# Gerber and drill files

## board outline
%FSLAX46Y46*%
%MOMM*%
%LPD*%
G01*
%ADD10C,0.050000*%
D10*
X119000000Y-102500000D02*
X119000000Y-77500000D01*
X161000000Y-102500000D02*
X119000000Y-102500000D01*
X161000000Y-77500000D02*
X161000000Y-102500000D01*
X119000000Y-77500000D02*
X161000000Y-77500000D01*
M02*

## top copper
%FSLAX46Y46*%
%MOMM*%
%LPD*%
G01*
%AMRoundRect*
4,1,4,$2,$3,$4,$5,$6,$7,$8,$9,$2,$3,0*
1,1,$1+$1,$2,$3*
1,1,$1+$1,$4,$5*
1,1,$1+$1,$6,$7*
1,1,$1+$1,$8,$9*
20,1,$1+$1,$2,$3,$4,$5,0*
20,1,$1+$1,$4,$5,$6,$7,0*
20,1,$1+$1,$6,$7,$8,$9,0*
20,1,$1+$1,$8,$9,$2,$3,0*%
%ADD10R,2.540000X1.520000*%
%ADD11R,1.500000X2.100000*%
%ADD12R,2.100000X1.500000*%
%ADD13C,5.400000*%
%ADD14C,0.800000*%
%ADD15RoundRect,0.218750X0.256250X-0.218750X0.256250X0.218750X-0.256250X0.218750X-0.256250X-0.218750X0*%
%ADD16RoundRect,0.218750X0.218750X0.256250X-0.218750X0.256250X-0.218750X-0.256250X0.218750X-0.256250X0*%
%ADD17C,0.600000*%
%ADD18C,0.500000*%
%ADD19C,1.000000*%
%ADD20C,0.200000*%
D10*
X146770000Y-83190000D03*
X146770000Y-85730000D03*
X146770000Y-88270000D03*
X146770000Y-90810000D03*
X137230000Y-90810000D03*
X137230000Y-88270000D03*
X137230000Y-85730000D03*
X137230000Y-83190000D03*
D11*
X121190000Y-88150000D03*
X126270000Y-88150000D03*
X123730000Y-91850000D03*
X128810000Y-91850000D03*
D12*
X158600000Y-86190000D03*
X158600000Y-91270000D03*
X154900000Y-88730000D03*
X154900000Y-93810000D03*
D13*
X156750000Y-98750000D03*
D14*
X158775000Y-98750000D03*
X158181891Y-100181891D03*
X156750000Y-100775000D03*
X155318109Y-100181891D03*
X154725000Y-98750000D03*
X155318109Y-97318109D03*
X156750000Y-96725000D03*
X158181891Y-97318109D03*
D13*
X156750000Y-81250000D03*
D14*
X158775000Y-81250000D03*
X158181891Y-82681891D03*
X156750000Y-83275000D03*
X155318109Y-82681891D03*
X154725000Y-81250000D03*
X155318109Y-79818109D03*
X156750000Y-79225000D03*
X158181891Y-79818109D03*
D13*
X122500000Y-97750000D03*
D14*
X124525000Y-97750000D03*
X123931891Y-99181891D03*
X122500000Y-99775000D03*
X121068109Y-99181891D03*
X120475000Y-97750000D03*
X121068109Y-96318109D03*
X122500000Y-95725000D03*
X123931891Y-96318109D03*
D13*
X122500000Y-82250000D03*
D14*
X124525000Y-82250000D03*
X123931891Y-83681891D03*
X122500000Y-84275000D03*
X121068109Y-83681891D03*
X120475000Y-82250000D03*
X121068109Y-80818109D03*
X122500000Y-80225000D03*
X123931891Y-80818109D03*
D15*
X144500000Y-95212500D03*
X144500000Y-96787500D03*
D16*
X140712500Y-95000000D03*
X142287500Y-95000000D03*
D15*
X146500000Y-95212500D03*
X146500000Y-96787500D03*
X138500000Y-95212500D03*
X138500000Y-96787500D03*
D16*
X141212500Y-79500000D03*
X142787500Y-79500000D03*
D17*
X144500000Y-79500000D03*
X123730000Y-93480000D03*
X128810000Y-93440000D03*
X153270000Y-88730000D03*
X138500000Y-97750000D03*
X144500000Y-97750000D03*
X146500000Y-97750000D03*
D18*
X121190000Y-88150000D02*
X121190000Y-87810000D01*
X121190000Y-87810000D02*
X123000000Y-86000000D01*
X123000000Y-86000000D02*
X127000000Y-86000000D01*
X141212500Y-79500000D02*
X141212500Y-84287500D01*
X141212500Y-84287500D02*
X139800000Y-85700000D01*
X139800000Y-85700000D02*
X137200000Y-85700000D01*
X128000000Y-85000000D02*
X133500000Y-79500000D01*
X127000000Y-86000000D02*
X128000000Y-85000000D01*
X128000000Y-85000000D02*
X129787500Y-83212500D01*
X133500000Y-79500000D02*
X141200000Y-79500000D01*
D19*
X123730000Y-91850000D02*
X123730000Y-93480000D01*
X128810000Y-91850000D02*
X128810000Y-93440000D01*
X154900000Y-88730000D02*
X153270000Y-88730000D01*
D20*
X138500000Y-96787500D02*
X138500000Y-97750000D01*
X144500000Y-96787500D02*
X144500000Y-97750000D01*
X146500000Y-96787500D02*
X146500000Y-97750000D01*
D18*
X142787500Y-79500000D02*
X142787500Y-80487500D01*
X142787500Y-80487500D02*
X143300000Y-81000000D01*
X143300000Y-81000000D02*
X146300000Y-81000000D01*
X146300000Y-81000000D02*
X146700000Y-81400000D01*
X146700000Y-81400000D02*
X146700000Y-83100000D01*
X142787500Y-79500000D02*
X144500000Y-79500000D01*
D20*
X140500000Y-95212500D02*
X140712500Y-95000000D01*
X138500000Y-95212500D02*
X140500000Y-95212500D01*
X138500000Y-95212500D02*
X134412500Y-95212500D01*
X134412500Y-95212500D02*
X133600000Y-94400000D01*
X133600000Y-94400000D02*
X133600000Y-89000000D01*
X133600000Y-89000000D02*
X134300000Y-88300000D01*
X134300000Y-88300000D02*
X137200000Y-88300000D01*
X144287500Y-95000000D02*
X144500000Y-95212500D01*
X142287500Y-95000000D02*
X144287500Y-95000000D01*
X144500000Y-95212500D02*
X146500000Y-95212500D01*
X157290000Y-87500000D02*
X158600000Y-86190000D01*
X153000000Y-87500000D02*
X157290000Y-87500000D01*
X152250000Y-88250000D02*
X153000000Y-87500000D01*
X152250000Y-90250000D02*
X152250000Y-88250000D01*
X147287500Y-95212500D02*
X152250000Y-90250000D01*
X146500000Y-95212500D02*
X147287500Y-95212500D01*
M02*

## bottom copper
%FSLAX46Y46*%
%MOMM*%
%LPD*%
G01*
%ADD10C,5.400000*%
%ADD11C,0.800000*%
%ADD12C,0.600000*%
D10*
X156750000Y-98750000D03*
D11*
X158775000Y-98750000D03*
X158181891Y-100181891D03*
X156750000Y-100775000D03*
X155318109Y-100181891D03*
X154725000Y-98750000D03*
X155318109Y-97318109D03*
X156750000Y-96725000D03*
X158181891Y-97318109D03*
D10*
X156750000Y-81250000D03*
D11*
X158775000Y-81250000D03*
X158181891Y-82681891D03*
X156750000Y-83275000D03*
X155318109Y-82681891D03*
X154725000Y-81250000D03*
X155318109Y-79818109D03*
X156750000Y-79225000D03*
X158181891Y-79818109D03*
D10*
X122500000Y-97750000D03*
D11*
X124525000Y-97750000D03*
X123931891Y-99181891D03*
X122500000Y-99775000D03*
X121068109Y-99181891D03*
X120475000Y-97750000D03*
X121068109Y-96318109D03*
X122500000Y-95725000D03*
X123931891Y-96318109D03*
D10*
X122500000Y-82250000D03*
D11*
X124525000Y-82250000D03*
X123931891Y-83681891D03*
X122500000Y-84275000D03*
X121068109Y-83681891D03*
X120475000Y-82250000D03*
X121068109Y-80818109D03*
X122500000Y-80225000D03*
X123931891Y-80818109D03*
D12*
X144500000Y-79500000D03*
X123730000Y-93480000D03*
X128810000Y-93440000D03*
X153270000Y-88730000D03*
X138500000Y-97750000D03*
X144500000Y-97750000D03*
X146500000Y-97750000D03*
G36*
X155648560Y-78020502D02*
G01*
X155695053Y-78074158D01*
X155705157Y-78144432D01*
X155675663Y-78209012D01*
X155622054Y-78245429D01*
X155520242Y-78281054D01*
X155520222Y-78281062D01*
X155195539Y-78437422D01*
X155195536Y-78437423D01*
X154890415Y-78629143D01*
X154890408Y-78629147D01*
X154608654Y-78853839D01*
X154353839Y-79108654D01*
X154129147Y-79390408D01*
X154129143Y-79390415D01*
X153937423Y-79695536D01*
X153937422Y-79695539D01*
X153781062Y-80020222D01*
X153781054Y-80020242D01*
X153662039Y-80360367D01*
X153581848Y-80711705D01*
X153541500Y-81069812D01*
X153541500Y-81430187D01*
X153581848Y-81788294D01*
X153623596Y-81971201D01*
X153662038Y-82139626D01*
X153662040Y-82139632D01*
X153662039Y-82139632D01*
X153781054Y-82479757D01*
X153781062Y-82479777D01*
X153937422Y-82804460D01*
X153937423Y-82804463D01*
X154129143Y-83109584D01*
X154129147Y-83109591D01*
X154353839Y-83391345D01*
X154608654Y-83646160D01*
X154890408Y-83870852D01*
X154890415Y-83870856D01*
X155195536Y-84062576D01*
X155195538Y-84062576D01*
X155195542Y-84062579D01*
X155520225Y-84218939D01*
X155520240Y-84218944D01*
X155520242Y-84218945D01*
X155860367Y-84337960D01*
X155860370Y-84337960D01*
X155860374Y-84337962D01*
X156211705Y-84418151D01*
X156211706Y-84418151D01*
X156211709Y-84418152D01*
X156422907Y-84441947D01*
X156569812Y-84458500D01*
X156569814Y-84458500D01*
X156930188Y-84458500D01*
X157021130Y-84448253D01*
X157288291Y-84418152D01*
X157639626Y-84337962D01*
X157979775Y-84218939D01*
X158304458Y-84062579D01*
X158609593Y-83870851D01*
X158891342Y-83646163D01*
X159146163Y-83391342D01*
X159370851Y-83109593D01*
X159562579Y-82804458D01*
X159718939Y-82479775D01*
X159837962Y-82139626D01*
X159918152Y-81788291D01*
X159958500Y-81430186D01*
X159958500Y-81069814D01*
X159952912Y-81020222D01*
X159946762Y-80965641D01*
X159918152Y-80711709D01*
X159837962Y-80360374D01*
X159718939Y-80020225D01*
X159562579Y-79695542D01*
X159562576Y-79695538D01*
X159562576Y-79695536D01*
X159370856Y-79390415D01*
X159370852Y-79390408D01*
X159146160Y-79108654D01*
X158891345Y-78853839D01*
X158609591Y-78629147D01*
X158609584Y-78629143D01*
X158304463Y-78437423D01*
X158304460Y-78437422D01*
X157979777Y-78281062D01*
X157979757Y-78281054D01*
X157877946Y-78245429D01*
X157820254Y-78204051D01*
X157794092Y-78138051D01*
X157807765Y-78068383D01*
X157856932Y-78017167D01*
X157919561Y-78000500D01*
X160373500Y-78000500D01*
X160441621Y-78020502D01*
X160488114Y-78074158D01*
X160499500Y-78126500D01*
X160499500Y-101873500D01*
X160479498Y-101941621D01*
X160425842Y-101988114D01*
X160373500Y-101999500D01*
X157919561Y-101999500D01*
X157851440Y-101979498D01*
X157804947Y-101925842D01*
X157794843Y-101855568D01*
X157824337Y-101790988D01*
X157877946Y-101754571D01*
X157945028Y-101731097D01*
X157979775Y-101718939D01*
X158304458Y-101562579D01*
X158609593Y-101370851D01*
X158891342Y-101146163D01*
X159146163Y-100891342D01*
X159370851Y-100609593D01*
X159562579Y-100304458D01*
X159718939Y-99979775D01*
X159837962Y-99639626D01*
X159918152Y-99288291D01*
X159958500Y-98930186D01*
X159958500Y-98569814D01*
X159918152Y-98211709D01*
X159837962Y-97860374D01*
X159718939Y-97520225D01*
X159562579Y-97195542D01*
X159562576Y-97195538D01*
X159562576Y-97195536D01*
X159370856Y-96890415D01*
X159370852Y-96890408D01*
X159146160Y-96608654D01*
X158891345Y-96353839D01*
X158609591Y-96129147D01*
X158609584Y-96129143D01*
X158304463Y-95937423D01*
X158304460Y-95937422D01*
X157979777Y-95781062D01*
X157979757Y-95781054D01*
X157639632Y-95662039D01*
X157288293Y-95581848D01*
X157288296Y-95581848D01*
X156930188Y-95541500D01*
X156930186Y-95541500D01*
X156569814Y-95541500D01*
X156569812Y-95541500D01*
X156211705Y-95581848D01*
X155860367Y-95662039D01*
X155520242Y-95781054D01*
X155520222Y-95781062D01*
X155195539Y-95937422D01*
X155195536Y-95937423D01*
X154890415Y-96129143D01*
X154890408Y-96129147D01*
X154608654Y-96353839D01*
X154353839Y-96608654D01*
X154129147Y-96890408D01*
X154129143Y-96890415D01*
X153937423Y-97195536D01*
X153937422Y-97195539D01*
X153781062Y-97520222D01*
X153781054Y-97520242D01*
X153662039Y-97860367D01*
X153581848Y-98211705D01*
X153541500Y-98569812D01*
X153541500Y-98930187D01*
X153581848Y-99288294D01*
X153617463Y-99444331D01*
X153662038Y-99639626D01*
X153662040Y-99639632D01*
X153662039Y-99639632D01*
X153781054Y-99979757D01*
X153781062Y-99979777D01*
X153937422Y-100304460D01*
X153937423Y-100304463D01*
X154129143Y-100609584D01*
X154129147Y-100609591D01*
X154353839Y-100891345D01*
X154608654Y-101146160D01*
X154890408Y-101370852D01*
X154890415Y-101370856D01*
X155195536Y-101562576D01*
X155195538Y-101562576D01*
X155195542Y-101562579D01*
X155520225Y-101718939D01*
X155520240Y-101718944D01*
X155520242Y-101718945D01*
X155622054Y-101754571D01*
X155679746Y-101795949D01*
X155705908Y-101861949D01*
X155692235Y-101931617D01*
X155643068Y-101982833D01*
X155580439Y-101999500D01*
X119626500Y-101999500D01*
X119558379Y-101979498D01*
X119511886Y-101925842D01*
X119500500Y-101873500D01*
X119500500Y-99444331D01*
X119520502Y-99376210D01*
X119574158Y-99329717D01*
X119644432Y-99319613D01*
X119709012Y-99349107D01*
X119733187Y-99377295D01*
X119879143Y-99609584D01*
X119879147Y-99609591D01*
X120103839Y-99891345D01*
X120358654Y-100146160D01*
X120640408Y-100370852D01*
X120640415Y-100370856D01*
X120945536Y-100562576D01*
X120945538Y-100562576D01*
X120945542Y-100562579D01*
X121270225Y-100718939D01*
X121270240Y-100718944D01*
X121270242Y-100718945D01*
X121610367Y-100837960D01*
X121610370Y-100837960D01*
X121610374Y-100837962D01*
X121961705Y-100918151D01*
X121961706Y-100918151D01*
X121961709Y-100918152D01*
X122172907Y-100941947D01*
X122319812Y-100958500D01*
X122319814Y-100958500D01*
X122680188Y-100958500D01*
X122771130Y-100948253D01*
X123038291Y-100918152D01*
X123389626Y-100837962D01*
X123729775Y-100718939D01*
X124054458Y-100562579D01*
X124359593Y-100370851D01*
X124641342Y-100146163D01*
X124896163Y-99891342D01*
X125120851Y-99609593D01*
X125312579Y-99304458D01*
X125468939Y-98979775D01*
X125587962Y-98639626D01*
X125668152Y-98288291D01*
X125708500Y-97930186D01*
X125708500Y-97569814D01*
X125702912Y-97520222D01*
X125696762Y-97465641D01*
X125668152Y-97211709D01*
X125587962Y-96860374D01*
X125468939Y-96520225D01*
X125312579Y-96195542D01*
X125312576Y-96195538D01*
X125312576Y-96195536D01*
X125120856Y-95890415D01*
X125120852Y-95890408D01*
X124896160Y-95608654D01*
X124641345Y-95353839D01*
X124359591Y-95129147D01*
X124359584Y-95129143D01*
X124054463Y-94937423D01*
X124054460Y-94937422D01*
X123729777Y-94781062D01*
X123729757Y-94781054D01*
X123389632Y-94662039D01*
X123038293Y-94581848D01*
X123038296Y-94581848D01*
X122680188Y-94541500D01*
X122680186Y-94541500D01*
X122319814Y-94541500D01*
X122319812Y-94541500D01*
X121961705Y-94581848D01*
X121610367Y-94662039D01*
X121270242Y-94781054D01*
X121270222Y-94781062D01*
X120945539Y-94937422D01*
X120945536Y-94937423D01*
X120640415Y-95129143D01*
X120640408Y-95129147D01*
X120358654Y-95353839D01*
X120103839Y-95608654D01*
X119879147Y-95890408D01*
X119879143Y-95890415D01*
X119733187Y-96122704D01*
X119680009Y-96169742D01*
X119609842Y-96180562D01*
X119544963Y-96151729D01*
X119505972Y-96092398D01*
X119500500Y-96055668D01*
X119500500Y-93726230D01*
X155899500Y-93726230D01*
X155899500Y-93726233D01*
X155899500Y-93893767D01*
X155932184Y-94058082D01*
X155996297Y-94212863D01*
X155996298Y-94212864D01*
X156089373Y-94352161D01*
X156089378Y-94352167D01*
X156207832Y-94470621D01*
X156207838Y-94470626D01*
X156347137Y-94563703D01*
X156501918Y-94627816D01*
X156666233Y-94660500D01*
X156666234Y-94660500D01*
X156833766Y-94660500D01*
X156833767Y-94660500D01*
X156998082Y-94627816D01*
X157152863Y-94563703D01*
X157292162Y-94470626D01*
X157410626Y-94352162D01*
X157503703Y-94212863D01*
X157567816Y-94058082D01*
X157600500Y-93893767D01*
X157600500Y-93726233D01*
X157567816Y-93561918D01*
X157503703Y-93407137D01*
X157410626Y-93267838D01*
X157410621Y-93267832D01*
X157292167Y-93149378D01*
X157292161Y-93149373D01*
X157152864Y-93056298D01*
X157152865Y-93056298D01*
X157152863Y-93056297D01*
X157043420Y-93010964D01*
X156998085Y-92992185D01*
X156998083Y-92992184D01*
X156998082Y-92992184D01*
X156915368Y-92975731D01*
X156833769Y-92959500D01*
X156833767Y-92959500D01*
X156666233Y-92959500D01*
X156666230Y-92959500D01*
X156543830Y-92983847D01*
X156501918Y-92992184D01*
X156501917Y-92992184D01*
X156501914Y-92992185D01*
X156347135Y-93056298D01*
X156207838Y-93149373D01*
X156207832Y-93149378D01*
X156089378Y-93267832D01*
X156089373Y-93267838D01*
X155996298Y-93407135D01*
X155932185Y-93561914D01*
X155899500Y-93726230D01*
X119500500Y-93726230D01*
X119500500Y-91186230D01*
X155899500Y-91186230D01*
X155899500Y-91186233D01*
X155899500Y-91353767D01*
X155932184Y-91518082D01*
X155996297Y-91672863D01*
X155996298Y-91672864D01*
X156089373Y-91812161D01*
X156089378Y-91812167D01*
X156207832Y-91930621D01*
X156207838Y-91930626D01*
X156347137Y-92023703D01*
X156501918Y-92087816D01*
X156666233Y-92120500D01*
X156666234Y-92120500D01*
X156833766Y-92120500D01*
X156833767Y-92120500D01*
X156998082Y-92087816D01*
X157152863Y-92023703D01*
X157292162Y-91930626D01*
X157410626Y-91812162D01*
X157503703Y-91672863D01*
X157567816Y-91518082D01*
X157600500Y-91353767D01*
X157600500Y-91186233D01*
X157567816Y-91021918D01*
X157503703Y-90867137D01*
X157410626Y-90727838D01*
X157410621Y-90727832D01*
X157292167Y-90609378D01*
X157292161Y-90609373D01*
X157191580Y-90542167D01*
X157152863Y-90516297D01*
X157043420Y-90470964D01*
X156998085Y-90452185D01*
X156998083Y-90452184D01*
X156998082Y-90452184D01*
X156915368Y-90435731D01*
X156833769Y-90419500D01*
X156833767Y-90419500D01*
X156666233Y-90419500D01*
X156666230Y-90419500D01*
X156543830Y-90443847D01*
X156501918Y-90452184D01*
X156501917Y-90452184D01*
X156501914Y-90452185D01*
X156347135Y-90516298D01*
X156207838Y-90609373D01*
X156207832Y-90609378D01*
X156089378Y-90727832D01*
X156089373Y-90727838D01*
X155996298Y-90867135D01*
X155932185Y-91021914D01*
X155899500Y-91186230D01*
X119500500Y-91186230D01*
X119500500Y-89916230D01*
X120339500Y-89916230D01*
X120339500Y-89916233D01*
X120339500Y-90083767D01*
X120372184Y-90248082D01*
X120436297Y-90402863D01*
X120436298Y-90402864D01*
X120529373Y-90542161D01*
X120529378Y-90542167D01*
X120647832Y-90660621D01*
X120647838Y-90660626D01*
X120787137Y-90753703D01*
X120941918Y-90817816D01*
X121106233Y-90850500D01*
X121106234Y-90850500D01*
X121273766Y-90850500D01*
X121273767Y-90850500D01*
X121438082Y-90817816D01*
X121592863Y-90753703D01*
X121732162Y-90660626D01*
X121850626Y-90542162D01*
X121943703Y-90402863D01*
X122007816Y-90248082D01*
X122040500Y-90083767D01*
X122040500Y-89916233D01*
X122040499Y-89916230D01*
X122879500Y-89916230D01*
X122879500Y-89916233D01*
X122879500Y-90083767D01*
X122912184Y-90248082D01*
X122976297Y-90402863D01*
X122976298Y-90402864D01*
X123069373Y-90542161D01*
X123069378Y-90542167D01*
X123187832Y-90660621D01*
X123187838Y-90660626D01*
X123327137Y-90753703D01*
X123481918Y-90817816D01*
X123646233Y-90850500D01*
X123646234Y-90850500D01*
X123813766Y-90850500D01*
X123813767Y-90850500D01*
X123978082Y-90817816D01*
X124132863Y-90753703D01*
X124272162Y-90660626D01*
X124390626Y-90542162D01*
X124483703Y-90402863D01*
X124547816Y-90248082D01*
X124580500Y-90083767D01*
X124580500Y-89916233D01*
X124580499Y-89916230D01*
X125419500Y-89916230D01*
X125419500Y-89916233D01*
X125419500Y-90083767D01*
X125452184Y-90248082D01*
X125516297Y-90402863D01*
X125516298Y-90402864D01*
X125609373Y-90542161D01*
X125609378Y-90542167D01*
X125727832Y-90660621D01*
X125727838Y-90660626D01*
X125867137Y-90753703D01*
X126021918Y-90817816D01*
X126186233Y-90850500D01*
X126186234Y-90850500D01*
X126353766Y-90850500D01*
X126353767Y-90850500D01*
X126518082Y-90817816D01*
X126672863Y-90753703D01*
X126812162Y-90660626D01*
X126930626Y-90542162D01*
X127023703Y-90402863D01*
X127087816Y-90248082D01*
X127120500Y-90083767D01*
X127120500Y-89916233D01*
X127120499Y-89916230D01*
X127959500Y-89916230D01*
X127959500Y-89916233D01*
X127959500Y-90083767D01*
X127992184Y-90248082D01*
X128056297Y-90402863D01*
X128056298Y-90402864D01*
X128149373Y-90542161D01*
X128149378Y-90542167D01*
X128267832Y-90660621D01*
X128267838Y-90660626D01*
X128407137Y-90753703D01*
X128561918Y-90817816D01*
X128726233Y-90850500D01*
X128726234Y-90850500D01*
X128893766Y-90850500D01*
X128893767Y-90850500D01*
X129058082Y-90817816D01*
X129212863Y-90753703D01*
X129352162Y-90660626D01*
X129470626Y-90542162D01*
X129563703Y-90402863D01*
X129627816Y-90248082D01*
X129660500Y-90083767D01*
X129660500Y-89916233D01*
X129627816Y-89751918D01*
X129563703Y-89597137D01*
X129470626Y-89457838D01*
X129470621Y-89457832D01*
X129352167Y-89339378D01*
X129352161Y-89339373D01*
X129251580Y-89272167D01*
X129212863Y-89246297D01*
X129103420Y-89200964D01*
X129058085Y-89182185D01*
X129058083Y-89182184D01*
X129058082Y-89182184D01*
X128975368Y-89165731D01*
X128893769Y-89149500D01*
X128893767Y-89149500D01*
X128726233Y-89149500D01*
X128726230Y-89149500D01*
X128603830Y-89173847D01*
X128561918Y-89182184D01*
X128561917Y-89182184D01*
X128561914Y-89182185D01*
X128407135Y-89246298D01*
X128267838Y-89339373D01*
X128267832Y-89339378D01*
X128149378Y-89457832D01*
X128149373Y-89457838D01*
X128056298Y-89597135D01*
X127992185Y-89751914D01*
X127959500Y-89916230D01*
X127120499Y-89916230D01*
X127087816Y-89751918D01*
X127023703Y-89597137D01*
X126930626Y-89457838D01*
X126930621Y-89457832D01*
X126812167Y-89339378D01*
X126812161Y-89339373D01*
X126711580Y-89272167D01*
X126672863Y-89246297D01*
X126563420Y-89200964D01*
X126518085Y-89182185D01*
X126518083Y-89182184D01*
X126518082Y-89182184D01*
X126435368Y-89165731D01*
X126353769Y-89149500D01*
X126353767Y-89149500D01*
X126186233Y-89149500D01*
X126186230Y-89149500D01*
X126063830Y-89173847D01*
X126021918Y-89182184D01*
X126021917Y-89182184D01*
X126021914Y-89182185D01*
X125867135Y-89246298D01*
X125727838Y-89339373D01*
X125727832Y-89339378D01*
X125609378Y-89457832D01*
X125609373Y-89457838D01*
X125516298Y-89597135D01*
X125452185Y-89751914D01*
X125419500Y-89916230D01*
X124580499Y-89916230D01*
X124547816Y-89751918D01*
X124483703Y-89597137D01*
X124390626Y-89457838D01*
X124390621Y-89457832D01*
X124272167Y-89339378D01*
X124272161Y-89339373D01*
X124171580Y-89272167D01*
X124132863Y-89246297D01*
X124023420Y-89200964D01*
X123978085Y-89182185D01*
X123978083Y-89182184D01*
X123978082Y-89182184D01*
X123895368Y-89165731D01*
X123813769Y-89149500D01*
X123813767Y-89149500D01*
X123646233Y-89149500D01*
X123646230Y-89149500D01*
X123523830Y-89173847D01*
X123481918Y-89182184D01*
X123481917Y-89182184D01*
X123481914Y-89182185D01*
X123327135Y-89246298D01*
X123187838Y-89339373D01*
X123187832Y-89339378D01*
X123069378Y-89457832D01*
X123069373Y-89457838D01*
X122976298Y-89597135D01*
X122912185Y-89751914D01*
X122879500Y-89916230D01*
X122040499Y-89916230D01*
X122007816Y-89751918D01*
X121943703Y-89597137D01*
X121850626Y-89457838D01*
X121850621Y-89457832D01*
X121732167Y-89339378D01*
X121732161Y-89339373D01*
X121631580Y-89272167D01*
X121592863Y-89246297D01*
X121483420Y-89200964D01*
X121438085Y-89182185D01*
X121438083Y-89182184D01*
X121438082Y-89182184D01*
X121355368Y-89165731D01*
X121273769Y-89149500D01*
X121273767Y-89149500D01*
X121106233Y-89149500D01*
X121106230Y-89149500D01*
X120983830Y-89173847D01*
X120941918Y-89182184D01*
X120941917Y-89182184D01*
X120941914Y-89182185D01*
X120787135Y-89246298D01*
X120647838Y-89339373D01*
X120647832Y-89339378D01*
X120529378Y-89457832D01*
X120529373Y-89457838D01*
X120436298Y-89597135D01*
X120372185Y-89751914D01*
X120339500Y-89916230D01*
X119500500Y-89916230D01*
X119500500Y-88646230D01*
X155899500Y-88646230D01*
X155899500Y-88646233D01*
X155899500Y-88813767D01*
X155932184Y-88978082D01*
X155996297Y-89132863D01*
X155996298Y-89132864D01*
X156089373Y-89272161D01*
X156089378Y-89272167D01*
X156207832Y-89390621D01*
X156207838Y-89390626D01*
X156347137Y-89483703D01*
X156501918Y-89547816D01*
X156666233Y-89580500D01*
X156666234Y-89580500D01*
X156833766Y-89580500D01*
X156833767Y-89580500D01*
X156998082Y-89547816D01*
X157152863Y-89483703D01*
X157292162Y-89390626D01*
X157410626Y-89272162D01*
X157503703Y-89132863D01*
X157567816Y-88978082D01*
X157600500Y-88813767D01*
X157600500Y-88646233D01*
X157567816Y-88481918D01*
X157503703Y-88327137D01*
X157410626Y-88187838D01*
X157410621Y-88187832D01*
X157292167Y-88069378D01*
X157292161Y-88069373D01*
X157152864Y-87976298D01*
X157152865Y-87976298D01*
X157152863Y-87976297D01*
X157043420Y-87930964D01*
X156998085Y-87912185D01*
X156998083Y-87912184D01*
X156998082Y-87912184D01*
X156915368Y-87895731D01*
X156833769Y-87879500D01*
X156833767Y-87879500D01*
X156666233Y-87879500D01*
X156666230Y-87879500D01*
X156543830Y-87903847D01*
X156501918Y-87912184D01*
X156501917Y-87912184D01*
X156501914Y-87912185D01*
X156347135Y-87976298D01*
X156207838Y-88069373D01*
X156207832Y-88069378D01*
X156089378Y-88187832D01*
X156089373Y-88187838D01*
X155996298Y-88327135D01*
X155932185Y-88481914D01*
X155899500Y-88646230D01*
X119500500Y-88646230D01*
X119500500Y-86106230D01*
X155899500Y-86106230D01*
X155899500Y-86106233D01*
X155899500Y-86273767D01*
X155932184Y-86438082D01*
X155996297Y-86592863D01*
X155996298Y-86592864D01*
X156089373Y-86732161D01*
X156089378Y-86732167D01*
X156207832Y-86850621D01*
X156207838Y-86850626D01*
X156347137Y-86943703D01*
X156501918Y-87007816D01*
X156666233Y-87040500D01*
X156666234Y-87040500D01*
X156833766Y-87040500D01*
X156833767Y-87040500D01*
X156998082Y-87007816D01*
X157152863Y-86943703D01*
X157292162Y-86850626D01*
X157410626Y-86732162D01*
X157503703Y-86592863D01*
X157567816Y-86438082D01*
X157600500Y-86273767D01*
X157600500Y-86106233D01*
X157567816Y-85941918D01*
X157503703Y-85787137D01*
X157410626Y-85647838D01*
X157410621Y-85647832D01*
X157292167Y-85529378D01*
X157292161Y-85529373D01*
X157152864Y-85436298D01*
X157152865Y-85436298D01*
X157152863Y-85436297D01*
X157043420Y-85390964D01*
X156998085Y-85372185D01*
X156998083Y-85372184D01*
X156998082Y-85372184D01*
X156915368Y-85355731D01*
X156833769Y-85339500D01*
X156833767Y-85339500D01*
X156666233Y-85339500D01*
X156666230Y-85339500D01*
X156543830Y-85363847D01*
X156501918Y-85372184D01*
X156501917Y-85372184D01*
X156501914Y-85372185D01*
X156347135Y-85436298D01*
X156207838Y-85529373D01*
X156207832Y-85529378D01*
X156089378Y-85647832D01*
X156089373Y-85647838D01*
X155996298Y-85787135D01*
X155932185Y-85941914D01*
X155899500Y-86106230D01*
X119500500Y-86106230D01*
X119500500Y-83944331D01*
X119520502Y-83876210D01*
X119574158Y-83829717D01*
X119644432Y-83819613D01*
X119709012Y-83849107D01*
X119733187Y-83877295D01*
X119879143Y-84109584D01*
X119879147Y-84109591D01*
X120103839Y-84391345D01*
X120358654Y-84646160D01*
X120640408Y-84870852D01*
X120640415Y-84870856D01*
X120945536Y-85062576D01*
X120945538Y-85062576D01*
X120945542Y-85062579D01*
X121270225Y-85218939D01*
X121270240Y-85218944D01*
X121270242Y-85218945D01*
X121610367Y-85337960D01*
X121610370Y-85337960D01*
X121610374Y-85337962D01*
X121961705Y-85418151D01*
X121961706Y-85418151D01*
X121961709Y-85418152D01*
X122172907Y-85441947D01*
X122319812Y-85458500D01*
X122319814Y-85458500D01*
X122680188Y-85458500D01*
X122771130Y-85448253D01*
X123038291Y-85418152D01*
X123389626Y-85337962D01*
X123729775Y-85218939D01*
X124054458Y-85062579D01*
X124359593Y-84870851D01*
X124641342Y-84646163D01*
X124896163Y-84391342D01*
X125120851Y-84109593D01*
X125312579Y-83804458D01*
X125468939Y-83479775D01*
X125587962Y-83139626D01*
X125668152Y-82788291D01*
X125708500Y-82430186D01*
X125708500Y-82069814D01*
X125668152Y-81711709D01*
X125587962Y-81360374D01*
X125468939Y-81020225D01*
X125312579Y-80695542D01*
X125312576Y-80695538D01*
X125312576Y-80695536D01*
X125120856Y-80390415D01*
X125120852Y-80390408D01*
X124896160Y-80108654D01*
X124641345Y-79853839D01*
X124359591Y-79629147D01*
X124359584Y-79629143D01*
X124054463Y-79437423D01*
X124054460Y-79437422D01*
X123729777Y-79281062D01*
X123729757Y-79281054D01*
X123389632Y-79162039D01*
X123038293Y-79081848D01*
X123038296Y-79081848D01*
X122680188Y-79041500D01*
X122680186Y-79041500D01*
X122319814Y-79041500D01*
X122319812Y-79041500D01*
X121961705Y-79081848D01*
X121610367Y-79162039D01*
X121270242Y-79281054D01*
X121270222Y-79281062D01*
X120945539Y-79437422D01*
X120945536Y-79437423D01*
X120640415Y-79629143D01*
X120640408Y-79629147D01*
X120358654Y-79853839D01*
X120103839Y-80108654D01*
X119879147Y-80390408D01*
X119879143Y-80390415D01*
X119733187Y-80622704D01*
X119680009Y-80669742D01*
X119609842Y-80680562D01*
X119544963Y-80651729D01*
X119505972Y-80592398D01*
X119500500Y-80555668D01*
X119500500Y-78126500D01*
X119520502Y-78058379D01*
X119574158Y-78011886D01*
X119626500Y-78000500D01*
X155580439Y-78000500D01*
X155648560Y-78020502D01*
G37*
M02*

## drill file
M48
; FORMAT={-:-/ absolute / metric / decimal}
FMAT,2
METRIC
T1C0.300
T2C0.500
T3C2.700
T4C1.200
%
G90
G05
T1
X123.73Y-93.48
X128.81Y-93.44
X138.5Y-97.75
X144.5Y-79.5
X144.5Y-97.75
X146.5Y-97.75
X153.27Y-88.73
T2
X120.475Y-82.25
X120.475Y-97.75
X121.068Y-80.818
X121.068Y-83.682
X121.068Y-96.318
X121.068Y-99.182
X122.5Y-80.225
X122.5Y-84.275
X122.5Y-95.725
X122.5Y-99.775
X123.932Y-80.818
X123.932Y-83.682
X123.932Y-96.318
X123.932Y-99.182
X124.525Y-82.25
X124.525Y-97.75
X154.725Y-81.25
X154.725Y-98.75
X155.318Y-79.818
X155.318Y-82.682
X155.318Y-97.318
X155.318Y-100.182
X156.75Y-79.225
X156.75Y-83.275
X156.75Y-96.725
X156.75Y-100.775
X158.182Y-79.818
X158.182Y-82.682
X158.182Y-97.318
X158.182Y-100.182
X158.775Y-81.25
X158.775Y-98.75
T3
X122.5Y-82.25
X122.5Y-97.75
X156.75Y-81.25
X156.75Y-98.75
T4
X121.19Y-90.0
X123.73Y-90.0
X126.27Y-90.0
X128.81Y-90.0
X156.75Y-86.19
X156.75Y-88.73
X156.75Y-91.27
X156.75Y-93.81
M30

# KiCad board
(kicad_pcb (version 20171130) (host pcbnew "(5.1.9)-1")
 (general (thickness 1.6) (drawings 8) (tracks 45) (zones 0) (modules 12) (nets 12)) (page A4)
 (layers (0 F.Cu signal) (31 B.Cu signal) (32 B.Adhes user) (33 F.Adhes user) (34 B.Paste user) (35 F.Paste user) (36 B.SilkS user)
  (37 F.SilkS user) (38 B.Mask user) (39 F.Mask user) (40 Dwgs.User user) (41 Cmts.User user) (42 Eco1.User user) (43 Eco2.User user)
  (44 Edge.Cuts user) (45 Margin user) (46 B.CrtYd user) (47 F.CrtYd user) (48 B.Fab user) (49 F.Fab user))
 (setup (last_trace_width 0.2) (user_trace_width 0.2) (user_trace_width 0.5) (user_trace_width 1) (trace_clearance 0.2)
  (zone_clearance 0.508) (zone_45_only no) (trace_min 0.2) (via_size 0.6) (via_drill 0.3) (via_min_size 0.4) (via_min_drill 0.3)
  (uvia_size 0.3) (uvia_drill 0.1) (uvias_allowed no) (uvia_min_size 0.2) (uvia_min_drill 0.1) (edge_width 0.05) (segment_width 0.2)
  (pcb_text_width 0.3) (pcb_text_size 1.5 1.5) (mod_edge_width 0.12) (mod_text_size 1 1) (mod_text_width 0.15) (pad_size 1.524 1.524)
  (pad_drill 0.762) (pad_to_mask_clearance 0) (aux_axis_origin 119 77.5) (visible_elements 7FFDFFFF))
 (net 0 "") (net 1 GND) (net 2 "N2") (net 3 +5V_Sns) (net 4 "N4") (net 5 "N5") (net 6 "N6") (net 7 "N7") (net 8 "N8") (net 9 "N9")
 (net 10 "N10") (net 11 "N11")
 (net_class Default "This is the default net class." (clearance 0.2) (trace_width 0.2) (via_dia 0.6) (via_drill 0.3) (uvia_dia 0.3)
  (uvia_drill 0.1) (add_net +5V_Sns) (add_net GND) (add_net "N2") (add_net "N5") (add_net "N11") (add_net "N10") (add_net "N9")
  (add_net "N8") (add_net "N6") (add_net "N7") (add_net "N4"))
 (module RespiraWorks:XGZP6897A (layer F.Cu) (at 142 87)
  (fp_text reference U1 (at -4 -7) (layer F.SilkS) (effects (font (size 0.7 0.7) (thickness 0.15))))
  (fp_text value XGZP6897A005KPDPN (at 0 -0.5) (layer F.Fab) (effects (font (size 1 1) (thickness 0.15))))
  (pad 8 smd rect (at 4.77 -3.81) (size 2.54 1.52) (layers F.Cu F.Paste F.Mask) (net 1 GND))
  (pad 7 smd rect (at 4.77 -1.27) (size 2.54 1.52) (layers F.Cu F.Paste F.Mask))
  (pad 6 smd rect (at 4.77 1.27) (size 2.54 1.52) (layers F.Cu F.Paste F.Mask))
  (pad 5 smd rect (at 4.77 3.81) (size 2.54 1.52) (layers F.Cu F.Paste F.Mask))
  (pad 4 smd rect (at -4.77 3.81) (size 2.54 1.52) (layers F.Cu F.Paste F.Mask))
  (pad 3 smd rect (at -4.77 1.27) (size 2.54 1.52) (layers F.Cu F.Paste F.Mask) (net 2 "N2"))
  (pad 2 smd rect (at -4.77 -1.27) (size 2.54 1.52) (layers F.Cu F.Paste F.Mask) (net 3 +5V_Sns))
  (pad 1 smd rect (at -4.77 -3.81) (size 2.54 1.52) (layers F.Cu F.Paste F.Mask)))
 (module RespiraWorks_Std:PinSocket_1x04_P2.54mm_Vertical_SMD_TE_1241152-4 (layer F.Cu) (at 125 90 90)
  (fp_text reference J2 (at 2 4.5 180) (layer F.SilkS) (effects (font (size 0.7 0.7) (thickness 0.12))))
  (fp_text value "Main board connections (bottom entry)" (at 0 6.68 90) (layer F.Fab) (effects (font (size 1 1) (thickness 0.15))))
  (pad "" np_thru_hole circle (at 0 1.27 90) (size 1.2 1.2) (drill 1.2) (layers *.Cu *.Mask))
  (pad "" np_thru_hole circle (at 0 -1.27 90) (size 1.2 1.2) (drill 1.2) (layers *.Cu *.Mask))
  (pad "" np_thru_hole circle (at 0 -3.81 90) (size 1.2 1.2) (drill 1.2) (layers *.Cu *.Mask))
  (pad 1 smd rect (at 1.85 -3.81 90) (size 2.1 1.5) (layers F.Cu F.Paste F.Mask) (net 3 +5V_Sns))
  (pad 3 smd rect (at 1.85 1.27 90) (size 2.1 1.5) (layers F.Cu F.Paste F.Mask) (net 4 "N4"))
  (pad 2 smd rect (at -1.85 -1.27 90) (size 2.1 1.5) (layers F.Cu F.Paste F.Mask) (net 1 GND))
  (pad 4 smd rect (at -1.85 3.81 90) (size 2.1 1.5) (layers F.Cu F.Paste F.Mask) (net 1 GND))
  (pad "" np_thru_hole circle (at 0 3.81 90) (size 1.2 1.2) (drill 1.2) (layers *.Cu *.Mask)))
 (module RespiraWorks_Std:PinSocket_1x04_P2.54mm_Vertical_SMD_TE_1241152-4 (layer F.Cu) (at 156.75 90)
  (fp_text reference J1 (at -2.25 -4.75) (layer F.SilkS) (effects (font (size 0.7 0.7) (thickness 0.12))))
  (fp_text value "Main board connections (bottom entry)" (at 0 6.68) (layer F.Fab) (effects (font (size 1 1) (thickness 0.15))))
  (pad "" np_thru_hole circle (at 0 1.27) (size 1.2 1.2) (drill 1.2) (layers *.Cu *.Mask))
  (pad "" np_thru_hole circle (at 0 -1.27) (size 1.2 1.2) (drill 1.2) (layers *.Cu *.Mask))
  (pad "" np_thru_hole circle (at 0 -3.81) (size 1.2 1.2) (drill 1.2) (layers *.Cu *.Mask))
  (pad 1 smd rect (at 1.85 -3.81) (size 2.1 1.5) (layers F.Cu F.Paste F.Mask) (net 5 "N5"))
  (pad 3 smd rect (at 1.85 1.27) (size 2.1 1.5) (layers F.Cu F.Paste F.Mask) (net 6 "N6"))
  (pad 2 smd rect (at -1.85 -1.27) (size 2.1 1.5) (layers F.Cu F.Paste F.Mask) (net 1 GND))
  (pad 4 smd rect (at -1.85 3.81) (size 2.1 1.5) (layers F.Cu F.Paste F.Mask) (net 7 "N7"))
  (pad "" np_thru_hole circle (at 0 3.81) (size 1.2 1.2) (drill 1.2) (layers *.Cu *.Mask)))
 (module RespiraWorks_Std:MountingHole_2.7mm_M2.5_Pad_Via (layer F.Cu) (at 156.75 98.75)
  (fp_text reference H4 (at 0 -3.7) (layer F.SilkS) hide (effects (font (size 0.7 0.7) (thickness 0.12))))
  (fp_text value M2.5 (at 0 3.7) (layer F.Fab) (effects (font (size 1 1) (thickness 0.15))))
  (pad 1 thru_hole circle (at 0 0) (size 5.4 5.4) (drill 2.7) (layers *.Cu *.Mask) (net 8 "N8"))
  (pad 1 thru_hole circle (at 2.025 0) (size 0.8 0.8) (drill 0.5) (layers *.Cu *.Mask) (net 8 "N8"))
  (pad 1 thru_hole circle (at 1.431891 1.431891) (size 0.8 0.8) (drill 0.5) (layers *.Cu *.Mask) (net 8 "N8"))
  (pad 1 thru_hole circle (at 0 2.025) (size 0.8 0.8) (drill 0.5) (layers *.Cu *.Mask) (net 8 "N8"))
  (pad 1 thru_hole circle (at -1.431891 1.431891) (size 0.8 0.8) (drill 0.5) (layers *.Cu *.Mask) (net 8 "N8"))
  (pad 1 thru_hole circle (at -2.025 0) (size 0.8 0.8) (drill 0.5) (layers *.Cu *.Mask) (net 8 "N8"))
  (pad 1 thru_hole circle (at -1.431891 -1.431891) (size 0.8 0.8) (drill 0.5) (layers *.Cu *.Mask) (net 8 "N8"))
  (pad 1 thru_hole circle (at 0 -2.025) (size 0.8 0.8) (drill 0.5) (layers *.Cu *.Mask) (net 8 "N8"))
  (pad 1 thru_hole circle (at 1.431891 -1.431891) (size 0.8 0.8) (drill 0.5) (layers *.Cu *.Mask) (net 8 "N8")))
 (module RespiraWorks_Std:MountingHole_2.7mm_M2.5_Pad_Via (layer F.Cu) (at 156.75 81.25)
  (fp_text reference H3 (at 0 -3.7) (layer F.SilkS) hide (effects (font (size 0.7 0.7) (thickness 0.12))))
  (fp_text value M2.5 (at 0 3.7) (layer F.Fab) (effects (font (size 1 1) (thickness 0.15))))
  (pad 1 thru_hole circle (at 0 0) (size 5.4 5.4) (drill 2.7) (layers *.Cu *.Mask) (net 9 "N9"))
  (pad 1 thru_hole circle (at 2.025 0) (size 0.8 0.8) (drill 0.5) (layers *.Cu *.Mask) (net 9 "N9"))
  (pad 1 thru_hole circle (at 1.431891 1.431891) (size 0.8 0.8) (drill 0.5) (layers *.Cu *.Mask) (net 9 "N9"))
  (pad 1 thru_hole circle (at 0 2.025) (size 0.8 0.8) (drill 0.5) (layers *.Cu *.Mask) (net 9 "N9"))
  (pad 1 thru_hole circle (at -1.431891 1.431891) (size 0.8 0.8) (drill 0.5) (layers *.Cu *.Mask) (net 9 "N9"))
  (pad 1 thru_hole circle (at -2.025 0) (size 0.8 0.8) (drill 0.5) (layers *.Cu *.Mask) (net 9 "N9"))
  (pad 1 thru_hole circle (at -1.431891 -1.431891) (size 0.8 0.8) (drill 0.5) (layers *.Cu *.Mask) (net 9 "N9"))
  (pad 1 thru_hole circle (at 0 -2.025) (size 0.8 0.8) (drill 0.5) (layers *.Cu *.Mask) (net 9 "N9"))
  (pad 1 thru_hole circle (at 1.431891 -1.431891) (size 0.8 0.8) (drill 0.5) (layers *.Cu *.Mask) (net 9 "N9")))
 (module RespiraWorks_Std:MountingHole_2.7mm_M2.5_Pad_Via (layer F.Cu) (at 122.5 97.75)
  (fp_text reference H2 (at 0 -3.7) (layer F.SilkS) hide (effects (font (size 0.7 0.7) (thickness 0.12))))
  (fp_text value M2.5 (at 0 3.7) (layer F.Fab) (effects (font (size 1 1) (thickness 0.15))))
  (pad 1 thru_hole circle (at 0 0) (size 5.4 5.4) (drill 2.7) (layers *.Cu *.Mask) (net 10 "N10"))
  (pad 1 thru_hole circle (at 2.025 0) (size 0.8 0.8) (drill 0.5) (layers *.Cu *.Mask) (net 10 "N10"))
  (pad 1 thru_hole circle (at 1.431891 1.431891) (size 0.8 0.8) (drill 0.5) (layers *.Cu *.Mask) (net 10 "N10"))
  (pad 1 thru_hole circle (at 0 2.025) (size 0.8 0.8) (drill 0.5) (layers *.Cu *.Mask) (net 10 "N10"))
  (pad 1 thru_hole circle (at -1.431891 1.431891) (size 0.8 0.8) (drill 0.5) (layers *.Cu *.Mask) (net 10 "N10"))
  (pad 1 thru_hole circle (at -2.025 0) (size 0.8 0.8) (drill 0.5) (layers *.Cu *.Mask) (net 10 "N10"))
  (pad 1 thru_hole circle (at -1.431891 -1.431891) (size 0.8 0.8) (drill 0.5) (layers *.Cu *.Mask) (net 10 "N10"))
  (pad 1 thru_hole circle (at 0 -2.025) (size 0.8 0.8) (drill 0.5) (layers *.Cu *.Mask) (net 10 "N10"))
  (pad 1 thru_hole circle (at 1.431891 -1.431891) (size 0.8 0.8) (drill 0.5) (layers *.Cu *.Mask) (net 10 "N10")))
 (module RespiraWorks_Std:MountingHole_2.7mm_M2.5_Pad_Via (layer F.Cu) (at 122.5 82.25)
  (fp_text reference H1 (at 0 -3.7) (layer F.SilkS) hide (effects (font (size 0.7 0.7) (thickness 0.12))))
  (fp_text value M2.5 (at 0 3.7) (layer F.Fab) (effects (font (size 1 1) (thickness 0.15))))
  (pad 1 thru_hole circle (at 0 0) (size 5.4 5.4) (drill 2.7) (layers *.Cu *.Mask) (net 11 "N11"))
  (pad 1 thru_hole circle (at 2.025 0) (size 0.8 0.8) (drill 0.5) (layers *.Cu *.Mask) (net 11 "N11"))
  (pad 1 thru_hole circle (at 1.431891 1.431891) (size 0.8 0.8) (drill 0.5) (layers *.Cu *.Mask) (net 11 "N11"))
  (pad 1 thru_hole circle (at 0 2.025) (size 0.8 0.8) (drill 0.5) (layers *.Cu *.Mask) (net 11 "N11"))
  (pad 1 thru_hole circle (at -1.431891 1.431891) (size 0.8 0.8) (drill 0.5) (layers *.Cu *.Mask) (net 11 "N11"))
  (pad 1 thru_hole circle (at -2.025 0) (size 0.8 0.8) (drill 0.5) (layers *.Cu *.Mask) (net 11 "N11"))
  (pad 1 thru_hole circle (at -1.431891 -1.431891) (size 0.8 0.8) (drill 0.5) (layers *.Cu *.Mask) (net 11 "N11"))
  (pad 1 thru_hole circle (at 0 -2.025) (size 0.8 0.8) (drill 0.5) (layers *.Cu *.Mask) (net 11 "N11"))
  (pad 1 thru_hole circle (at 1.431891 -1.431891) (size 0.8 0.8) (drill 0.5) (layers *.Cu *.Mask) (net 11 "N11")))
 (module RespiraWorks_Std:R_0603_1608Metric (layer F.Cu) (at 144.5 96 90)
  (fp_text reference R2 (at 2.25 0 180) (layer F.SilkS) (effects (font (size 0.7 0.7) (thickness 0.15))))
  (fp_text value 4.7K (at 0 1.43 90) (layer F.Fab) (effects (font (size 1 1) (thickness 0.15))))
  (pad 2 smd roundrect (at 0.7875 0 90) (size 0.875 0.95) (layers F.Cu F.Paste F.Mask) (roundrect_rratio 0.25) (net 5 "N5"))
  (pad 1 smd roundrect (at -0.7875 0 90) (size 0.875 0.95) (layers F.Cu F.Paste F.Mask) (roundrect_rratio 0.25) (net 1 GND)))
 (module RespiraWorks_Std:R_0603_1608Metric (layer F.Cu) (at 141.5 95 180)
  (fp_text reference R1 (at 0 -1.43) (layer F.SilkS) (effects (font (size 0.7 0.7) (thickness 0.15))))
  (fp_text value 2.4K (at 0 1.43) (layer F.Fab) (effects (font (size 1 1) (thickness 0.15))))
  (pad 2 smd roundrect (at 0.7875 0 180) (size 0.875 0.95) (layers F.Cu F.Paste F.Mask) (roundrect_rratio 0.25) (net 2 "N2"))
  (pad 1 smd roundrect (at -0.7875 0 180) (size 0.875 0.95) (layers F.Cu F.Paste F.Mask) (roundrect_rratio 0.25) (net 5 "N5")))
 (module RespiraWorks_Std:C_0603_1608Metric (layer F.Cu) (at 146.5 96 90)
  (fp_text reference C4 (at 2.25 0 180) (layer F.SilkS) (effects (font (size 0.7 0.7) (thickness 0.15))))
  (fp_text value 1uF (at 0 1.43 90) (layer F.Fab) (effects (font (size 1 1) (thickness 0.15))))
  (pad 2 smd roundrect (at 0.7875 0 90) (size 0.875 0.95) (layers F.Cu F.Paste F.Mask) (roundrect_rratio 0.25) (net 5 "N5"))
  (pad 1 smd roundrect (at -0.7875 0 90) (size 0.875 0.95) (layers F.Cu F.Paste F.Mask) (roundrect_rratio 0.25) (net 1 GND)))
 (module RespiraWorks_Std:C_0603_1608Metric (layer F.Cu) (at 138.5 96 90)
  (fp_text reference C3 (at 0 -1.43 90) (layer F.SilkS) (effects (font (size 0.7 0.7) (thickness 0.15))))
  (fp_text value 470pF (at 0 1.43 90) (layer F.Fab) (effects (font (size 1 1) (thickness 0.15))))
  (pad 2 smd roundrect (at 0.7875 0 90) (size 0.875 0.95) (layers F.Cu F.Paste F.Mask) (roundrect_rratio 0.25) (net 2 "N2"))
  (pad 1 smd roundrect (at -0.7875 0 90) (size 0.875 0.95) (layers F.Cu F.Paste F.Mask) (roundrect_rratio 0.25) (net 1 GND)))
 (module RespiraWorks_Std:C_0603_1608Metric (layer F.Cu) (at 142 79.5 180)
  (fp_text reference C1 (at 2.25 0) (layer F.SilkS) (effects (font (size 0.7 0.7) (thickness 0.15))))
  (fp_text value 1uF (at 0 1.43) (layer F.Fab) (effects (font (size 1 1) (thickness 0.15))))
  (pad 2 smd roundrect (at 0.7875 0 180) (size 0.875 0.95) (layers F.Cu F.Paste F.Mask) (roundrect_rratio 0.25) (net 3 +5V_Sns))
  (pad 1 smd roundrect (at -0.7875 0 180) (size 0.875 0.95) (layers F.Cu F.Paste F.Mask) (roundrect_rratio 0.25) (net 1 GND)))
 (gr_line (start 119 102.5) (end 119 77.5) (layer Edge.Cuts) (width 0.05))
 (gr_line (start 161 102.5) (end 119 102.5) (layer Edge.Cuts) (width 0.05))
 (gr_line (start 161 77.5) (end 161 102.5) (layer Edge.Cuts) (width 0.05))
 (gr_line (start 119 77.5) (end 161 77.5) (layer Edge.Cuts) (width 0.05))
 (segment (start 121.19 88.15) (end 121.19 87.81) (width 0.5) (layer F.Cu) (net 3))
 (segment (start 121.19 87.81) (end 123 86) (width 0.5) (layer F.Cu) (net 3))
 (segment (start 123 86) (end 127 86) (width 0.5) (layer F.Cu) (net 3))
 (segment (start 141.2125 79.5) (end 141.2125 84.2875) (width 0.5) (layer F.Cu) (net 3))
 (segment (start 141.2125 84.2875) (end 139.8 85.7) (width 0.5) (layer F.Cu) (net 3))
 (segment (start 139.8 85.7) (end 137.2 85.7) (width 0.5) (layer F.Cu) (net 3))
 (segment (start 128 85) (end 133.5 79.5) (width 0.5) (layer F.Cu) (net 3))
 (segment (start 127 86) (end 128 85) (width 0.5) (layer F.Cu) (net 3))
 (segment (start 128 85) (end 129.7875 83.2125) (width 0.5) (layer F.Cu) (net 3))
 (segment (start 133.5 79.5) (end 141.2 79.5) (width 0.5) (layer F.Cu) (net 3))
 (via (at 144.5 79.5) (size 0.6) (drill 0.3) (layers F.Cu B.Cu) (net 1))
 (segment (start 123.73 91.85) (end 123.73 93.48) (width 1) (layer F.Cu) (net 1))
 (via (at 123.73 93.48) (size 0.6) (drill 0.3) (layers F.Cu B.Cu) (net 1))
 (segment (start 128.81 91.85) (end 128.81 93.44) (width 1) (layer F.Cu) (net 1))
 (via (at 128.81 93.44) (size 0.6) (drill 0.3) (layers F.Cu B.Cu) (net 1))
 (segment (start 154.9 88.73) (end 153.27 88.73) (width 1) (layer F.Cu) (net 1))
 (via (at 153.27 88.73) (size 0.6) (drill 0.3) (layers F.Cu B.Cu) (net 1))
 (segment (start 138.5 96.7875) (end 138.5 97.75) (width 0.2) (layer F.Cu) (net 1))
 (via (at 138.5 97.75) (size 0.6) (drill 0.3) (layers F.Cu B.Cu) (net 1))
 (segment (start 144.5 96.7875) (end 144.5 97.75) (width 0.2) (layer F.Cu) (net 1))
 (via (at 144.5 97.75) (size 0.6) (drill 0.3) (layers F.Cu B.Cu) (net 1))
 (segment (start 146.5 96.7875) (end 146.5 97.75) (width 0.2) (layer F.Cu) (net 1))
 (via (at 146.5 97.75) (size 0.6) (drill 0.3) (layers F.Cu B.Cu) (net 1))
 (segment (start 142.7875 79.5) (end 142.7875 80.4875) (width 0.5) (layer F.Cu) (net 1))
 (segment (start 142.7875 80.4875) (end 143.3 81) (width 0.5) (layer F.Cu) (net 1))
 (segment (start 143.3 81) (end 146.3 81) (width 0.5) (layer F.Cu) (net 1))
 (segment (start 146.3 81) (end 146.7 81.4) (width 0.5) (layer F.Cu) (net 1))
 (segment (start 146.7 81.4) (end 146.7 83.1) (width 0.5) (layer F.Cu) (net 1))
 (segment (start 142.7875 79.5) (end 144.5 79.5) (width 0.5) (layer F.Cu) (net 1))
 (segment (start 140.5 95.2125) (end 140.7125 95) (width 0.2) (layer F.Cu) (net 2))
 (segment (start 138.5 95.2125) (end 140.5 95.2125) (width 0.2) (layer F.Cu) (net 2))
 (segment (start 138.5 95.2125) (end 134.4125 95.2125) (width 0.2) (layer F.Cu) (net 2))
 (segment (start 134.4125 95.2125) (end 133.6 94.4) (width 0.2) (layer F.Cu) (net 2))
 (segment (start 133.6 94.4) (end 133.6 89) (width 0.2) (layer F.Cu) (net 2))
 (segment (start 133.6 89) (end 134.3 88.3) (width 0.2) (layer F.Cu) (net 2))
 (segment (start 134.3 88.3) (end 137.2 88.3) (width 0.2) (layer F.Cu) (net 2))
 (segment (start 144.2875 95) (end 144.5 95.2125) (width 0.2) (layer F.Cu) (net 5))
 (segment (start 142.2875 95) (end 144.2875 95) (width 0.2) (layer F.Cu) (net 5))
 (segment (start 144.5 95.2125) (end 146.5 95.2125) (width 0.2) (layer F.Cu) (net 5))
 (segment (start 157.29 87.5) (end 158.6 86.19) (width 0.2) (layer F.Cu) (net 5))
 (segment (start 153 87.5) (end 157.29 87.5) (width 0.2) (layer F.Cu) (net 5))
 (segment (start 152.25 88.25) (end 153 87.5) (width 0.2) (layer F.Cu) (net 5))
 (segment (start 152.25 90.25) (end 152.25 88.25) (width 0.2) (layer F.Cu) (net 5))
 (segment (start 147.2875 95.2125) (end 152.25 90.25) (width 0.2) (layer F.Cu) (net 5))
 (segment (start 146.5 95.2125) (end 147.2875 95.2125) (width 0.2) (layer F.Cu) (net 5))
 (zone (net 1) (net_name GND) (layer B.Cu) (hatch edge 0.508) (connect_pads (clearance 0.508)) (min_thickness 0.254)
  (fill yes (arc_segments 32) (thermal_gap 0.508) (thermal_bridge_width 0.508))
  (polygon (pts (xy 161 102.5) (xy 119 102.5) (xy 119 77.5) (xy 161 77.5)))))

